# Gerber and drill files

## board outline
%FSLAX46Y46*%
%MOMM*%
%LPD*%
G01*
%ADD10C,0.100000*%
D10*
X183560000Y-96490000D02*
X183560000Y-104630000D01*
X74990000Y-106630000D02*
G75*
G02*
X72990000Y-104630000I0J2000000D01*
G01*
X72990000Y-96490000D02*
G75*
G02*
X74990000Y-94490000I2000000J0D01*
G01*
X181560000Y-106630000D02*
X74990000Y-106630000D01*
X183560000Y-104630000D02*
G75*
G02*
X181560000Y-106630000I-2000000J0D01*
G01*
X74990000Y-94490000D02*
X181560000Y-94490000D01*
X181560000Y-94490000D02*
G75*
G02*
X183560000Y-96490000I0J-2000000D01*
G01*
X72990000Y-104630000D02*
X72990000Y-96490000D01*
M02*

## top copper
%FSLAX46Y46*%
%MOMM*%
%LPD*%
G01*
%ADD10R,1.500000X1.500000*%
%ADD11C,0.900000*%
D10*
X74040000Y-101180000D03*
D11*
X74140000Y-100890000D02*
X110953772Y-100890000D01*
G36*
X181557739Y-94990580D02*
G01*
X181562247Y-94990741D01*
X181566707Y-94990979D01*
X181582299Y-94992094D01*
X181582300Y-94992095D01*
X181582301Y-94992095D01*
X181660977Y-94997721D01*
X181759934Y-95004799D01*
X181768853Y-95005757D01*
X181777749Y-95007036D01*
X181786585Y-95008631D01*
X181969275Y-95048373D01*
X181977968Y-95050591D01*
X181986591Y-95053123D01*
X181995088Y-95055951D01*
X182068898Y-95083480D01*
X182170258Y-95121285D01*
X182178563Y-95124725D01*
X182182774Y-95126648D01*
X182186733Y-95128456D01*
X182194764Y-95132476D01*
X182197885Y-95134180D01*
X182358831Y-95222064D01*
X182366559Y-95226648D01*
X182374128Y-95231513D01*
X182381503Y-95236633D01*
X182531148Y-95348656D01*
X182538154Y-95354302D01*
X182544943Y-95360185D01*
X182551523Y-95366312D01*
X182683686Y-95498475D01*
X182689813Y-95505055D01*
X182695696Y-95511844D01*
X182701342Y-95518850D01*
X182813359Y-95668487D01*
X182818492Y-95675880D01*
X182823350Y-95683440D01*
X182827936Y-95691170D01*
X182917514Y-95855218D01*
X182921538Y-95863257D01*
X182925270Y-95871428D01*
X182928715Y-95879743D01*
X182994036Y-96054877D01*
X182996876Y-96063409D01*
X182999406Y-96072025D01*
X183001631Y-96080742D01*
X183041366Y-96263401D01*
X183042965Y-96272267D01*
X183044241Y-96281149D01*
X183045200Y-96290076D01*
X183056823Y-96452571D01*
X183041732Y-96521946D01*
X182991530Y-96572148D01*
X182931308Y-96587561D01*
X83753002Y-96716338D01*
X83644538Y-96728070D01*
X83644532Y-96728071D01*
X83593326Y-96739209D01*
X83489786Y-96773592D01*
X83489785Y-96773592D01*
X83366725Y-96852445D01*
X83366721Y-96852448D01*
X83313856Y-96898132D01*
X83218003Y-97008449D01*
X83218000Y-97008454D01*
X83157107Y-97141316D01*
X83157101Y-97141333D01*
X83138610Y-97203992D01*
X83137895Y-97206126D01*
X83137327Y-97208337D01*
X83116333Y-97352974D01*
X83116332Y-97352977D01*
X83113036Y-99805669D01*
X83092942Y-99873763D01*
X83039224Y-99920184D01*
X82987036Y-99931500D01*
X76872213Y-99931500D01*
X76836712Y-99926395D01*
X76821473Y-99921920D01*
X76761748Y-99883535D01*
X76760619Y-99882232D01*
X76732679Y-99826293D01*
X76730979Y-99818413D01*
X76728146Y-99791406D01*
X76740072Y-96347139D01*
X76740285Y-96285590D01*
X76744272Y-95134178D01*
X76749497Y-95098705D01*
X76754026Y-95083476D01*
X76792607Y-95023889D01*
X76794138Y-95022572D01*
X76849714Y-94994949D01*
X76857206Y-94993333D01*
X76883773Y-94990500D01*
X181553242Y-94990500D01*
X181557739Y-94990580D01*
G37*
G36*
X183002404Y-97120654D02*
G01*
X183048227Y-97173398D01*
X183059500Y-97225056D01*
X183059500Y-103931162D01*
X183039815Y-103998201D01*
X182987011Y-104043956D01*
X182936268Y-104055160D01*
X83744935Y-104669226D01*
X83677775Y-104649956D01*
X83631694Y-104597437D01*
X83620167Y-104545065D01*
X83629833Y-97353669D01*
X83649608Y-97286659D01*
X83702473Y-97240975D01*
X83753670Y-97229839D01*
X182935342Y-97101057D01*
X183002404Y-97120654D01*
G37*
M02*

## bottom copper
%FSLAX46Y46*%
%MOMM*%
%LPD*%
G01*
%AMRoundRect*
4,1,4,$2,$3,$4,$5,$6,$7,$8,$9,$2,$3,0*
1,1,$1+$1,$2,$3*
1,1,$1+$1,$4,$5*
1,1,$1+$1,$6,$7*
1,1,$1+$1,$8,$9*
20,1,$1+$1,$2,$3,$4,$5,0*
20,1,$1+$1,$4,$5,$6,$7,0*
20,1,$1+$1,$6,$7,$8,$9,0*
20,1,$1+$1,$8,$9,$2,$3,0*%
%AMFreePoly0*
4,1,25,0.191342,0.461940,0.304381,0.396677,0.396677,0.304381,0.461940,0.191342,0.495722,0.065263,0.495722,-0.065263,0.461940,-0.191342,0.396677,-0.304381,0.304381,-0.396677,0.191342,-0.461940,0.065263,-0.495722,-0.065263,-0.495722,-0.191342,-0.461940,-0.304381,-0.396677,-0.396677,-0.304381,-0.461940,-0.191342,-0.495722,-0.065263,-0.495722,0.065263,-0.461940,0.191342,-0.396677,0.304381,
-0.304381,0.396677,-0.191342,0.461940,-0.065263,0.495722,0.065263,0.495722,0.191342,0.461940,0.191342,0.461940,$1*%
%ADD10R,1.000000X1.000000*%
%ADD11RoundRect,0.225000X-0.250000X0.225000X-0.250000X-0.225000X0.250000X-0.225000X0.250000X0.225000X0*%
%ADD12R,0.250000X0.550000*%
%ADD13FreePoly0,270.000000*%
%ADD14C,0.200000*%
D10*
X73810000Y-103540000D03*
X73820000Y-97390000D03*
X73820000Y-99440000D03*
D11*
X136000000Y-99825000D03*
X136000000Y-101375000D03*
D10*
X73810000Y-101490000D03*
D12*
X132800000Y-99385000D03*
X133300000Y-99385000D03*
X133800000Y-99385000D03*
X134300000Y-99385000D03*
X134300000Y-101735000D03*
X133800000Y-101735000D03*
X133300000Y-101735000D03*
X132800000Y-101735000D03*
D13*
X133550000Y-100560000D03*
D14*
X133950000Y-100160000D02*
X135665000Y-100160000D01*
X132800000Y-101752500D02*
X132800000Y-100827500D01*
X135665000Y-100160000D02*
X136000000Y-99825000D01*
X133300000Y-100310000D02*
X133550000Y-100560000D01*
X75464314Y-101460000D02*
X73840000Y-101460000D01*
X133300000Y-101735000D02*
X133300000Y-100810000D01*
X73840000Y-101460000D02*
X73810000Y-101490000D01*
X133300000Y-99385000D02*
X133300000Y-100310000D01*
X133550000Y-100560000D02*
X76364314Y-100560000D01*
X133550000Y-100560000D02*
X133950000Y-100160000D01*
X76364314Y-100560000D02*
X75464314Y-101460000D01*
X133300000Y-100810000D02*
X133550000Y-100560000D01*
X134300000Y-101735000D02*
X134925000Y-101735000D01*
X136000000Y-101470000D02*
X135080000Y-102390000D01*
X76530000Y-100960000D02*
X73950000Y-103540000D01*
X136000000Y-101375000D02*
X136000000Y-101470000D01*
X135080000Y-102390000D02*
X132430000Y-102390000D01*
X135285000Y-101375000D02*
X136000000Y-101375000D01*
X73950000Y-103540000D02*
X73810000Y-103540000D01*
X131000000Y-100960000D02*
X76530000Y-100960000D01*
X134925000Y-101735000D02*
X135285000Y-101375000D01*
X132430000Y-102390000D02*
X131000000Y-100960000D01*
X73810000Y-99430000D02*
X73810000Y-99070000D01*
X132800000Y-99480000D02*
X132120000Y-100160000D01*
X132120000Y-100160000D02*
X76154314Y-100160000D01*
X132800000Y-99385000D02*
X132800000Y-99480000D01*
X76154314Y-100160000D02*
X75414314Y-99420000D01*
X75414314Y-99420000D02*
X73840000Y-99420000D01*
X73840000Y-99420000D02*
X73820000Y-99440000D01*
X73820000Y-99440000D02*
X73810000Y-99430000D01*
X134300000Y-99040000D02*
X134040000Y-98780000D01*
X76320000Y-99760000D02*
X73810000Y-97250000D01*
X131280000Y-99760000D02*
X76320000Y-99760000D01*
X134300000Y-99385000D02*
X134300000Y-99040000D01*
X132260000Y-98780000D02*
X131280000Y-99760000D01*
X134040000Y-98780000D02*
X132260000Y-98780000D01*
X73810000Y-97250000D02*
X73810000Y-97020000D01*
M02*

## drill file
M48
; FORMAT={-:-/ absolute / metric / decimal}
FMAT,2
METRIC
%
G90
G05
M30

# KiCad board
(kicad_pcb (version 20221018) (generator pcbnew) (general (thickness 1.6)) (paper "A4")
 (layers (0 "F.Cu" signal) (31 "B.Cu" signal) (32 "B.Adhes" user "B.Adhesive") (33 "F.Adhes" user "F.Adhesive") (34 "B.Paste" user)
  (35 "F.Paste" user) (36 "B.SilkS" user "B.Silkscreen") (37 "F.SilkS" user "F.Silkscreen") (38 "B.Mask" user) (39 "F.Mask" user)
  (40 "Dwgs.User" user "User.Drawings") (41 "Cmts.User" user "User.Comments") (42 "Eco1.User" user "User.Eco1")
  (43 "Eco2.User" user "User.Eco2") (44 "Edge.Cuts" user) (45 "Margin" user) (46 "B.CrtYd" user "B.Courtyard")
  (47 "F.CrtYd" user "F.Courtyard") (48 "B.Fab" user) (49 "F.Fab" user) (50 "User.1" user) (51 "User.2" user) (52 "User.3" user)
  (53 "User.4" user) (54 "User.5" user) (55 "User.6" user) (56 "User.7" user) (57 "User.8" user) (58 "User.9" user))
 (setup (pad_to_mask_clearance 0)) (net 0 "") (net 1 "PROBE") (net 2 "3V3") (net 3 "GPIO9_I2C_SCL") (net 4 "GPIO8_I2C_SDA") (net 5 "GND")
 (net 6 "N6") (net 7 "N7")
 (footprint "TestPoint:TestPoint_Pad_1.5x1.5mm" (layer "F.Cu") (at 74.04 101.18)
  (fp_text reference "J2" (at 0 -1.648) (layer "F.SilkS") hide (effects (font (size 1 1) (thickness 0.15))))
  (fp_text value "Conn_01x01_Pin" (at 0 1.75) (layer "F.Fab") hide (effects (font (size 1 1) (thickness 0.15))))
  (pad "1" smd rect (at 0 0) (size 1.5 1.5) (layers "F.Cu" "F.Mask") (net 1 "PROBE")))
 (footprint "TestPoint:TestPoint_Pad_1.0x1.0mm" (layer "B.Cu") (at 73.81 103.54 180)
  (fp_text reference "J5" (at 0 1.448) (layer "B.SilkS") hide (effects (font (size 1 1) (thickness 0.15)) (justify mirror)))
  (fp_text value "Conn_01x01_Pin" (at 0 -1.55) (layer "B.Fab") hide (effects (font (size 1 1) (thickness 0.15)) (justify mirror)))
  (pad "1" smd rect (at 0 0 180) (size 1 1) (layers "B.Cu" "B.Mask") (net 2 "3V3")))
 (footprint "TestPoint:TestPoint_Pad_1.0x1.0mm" (layer "B.Cu") (at 73.82 97.39 180)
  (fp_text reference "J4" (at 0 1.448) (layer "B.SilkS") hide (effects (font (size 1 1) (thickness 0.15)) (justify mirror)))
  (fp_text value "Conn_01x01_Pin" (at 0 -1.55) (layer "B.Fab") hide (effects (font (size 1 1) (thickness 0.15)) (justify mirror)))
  (pad "1" smd rect (at 0 0 180) (size 1 1) (layers "B.Cu" "B.Mask") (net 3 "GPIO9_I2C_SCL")))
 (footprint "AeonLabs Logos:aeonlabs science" (layer "B.Cu") (at 174.289702 100.771553)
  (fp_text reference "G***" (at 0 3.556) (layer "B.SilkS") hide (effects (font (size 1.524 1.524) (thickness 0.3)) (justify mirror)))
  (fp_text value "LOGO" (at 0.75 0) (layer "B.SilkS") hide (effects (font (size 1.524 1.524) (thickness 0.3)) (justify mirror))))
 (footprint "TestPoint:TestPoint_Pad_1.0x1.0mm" (layer "B.Cu") (at 73.82 99.44 180)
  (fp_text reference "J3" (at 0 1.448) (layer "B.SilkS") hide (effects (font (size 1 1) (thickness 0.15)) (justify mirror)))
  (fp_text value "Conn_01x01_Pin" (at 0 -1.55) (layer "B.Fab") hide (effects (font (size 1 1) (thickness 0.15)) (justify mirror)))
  (pad "1" smd rect (at 0 0 180) (size 1 1) (layers "B.Cu" "B.Mask") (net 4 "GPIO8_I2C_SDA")))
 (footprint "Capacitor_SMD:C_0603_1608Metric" (layer "B.Cu") (at 136 100.6 -90)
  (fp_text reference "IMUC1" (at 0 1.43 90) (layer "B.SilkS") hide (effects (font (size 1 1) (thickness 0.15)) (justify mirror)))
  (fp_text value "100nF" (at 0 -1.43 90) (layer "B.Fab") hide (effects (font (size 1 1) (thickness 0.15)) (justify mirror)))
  (pad "1" smd roundrect (at -0.775 0 270) (size 0.9 0.95) (layers "B.Cu" "B.Paste" "B.Mask") (roundrect_rratio 0.25) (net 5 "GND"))
  (pad "2" smd roundrect (at 0.775 0 270) (size 0.9 0.95) (layers "B.Cu" "B.Paste" "B.Mask") (roundrect_rratio 0.25) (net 2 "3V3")))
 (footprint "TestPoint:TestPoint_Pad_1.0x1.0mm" (layer "B.Cu") (at 73.81 101.49 180)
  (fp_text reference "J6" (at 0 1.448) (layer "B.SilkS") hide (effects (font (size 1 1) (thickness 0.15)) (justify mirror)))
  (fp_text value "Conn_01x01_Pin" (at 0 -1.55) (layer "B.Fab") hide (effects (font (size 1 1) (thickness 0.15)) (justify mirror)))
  (pad "1" smd rect (at 0 0 180) (size 1 1) (layers "B.Cu" "B.Mask") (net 5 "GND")))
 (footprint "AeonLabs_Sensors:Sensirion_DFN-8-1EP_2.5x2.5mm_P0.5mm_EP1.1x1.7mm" (layer "B.Cu") (at 133.55 100.56 -90)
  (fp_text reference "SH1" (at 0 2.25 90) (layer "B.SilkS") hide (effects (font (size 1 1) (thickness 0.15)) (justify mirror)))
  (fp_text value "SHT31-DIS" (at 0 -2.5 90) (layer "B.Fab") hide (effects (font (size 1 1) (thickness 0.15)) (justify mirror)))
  (pad "" smd custom (at 0 0 270) (size 0.9 0.9) (layers "B.Paste") (zone_connect 0) (thermal_bridge_angle 45)
   (options (clearance outline) (anchor rect)) (primitives))
  (pad "1" smd rect (at -1.175 0.75 270) (size 0.55 0.25) (layers "B.Cu" "B.Paste" "B.Mask") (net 4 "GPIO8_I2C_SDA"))
  (pad "2" smd rect (at -1.175 0.25 270) (size 0.55 0.25) (layers "B.Cu" "B.Paste" "B.Mask") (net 5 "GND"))
  (pad "3" smd rect (at -1.175 -0.25 270) (size 0.55 0.25) (layers "B.Cu" "B.Paste" "B.Mask") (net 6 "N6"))
  (pad "4" smd rect (at -1.175 -0.75 90) (size 0.55 0.25) (layers "B.Cu" "B.Paste" "B.Mask") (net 3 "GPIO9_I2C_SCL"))
  (pad "5" smd rect (at 1.175 -0.75 270) (size 0.55 0.25) (layers "B.Cu" "B.Paste" "B.Mask") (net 2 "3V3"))
  (pad "6" smd rect (at 1.175 -0.25 270) (size 0.55 0.25) (layers "B.Cu" "B.Paste" "B.Mask") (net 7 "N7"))
  (pad "7" smd rect (at 1.175 0.25 270) (size 0.55 0.25) (layers "B.Cu" "B.Paste" "B.Mask") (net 5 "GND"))
  (pad "8" smd rect (at 1.175 0.75 270) (size 0.55 0.25) (layers "B.Cu" "B.Paste" "B.Mask") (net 5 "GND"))
  (pad "9" smd custom (at 0 0 270) (size 1 1) (layers "B.Cu" "B.Mask") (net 5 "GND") (zone_connect 0) (thermal_bridge_angle 45)
   (options (clearance outline) (anchor circle)) (primitives)))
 (gr_line (start 183.56 96.49) (end 183.56 104.63) (stroke (width 0.1) (type default)) (layer "Edge.Cuts"))
 (gr_arc (start 74.99 106.63) (mid 73.575786 106.044214) (end 72.99 104.63) (stroke (width 0.1) (type default)) (layer "Edge.Cuts"))
 (gr_arc (start 72.99 96.49) (mid 73.575786 95.075786) (end 74.99 94.49) (stroke (width 0.1) (type default)) (layer "Edge.Cuts"))
 (gr_line (start 181.56 106.63) (end 74.99 106.63) (stroke (width 0.1) (type default)) (layer "Edge.Cuts"))
 (gr_arc (start 183.56 104.63) (mid 182.974214 106.044214) (end 181.56 106.63) (stroke (width 0.1) (type default)) (layer "Edge.Cuts"))
 (gr_line (start 74.99 94.49) (end 181.56 94.49) (stroke (width 0.1) (type default)) (layer "Edge.Cuts"))
 (gr_arc (start 181.56 94.49) (mid 182.974214 95.075786) (end 183.56 96.49) (stroke (width 0.1) (type default)) (layer "Edge.Cuts"))
 (gr_line (start 72.99 104.63) (end 72.99 96.49) (stroke (width 0.1) (type default)) (layer "Edge.Cuts"))
 (segment (start 74.14 100.89) (end 110.953772 100.89) (width 0.9) (layer "F.Cu") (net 1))
 (segment (start 133.95 100.16) (end 135.665 100.16) (width 0.2) (layer "B.Cu") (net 5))
 (segment (start 132.8 101.7525) (end 132.8 100.8275) (width 0.2) (layer "B.Cu") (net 5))
 (segment (start 135.665 100.16) (end 136 99.825) (width 0.2) (layer "B.Cu") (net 5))
 (segment (start 133.3 100.31) (end 133.55 100.56) (width 0.2) (layer "B.Cu") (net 5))
 (segment (start 75.464314 101.46) (end 73.84 101.46) (width 0.2) (layer "B.Cu") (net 5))
 (segment (start 133.3 101.735) (end 133.3 100.81) (width 0.2) (layer "B.Cu") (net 5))
 (segment (start 73.84 101.46) (end 73.81 101.49) (width 0.2) (layer "B.Cu") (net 5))
 (segment (start 133.3 99.385) (end 133.3 100.31) (width 0.2) (layer "B.Cu") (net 5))
 (segment (start 133.55 100.56) (end 76.364314 100.56) (width 0.2) (layer "B.Cu") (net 5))
 (segment (start 133.55 100.56) (end 133.95 100.16) (width 0.2) (layer "B.Cu") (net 5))
 (segment (start 76.364314 100.56) (end 75.464314 101.46) (width 0.2) (layer "B.Cu") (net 5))
 (segment (start 133.3 100.81) (end 133.55 100.56) (width 0.2) (layer "B.Cu") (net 5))
 (segment (start 134.3 101.735) (end 134.925 101.735) (width 0.2) (layer "B.Cu") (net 2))
 (segment (start 136 101.47) (end 135.08 102.39) (width 0.2) (layer "B.Cu") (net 2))
 (segment (start 76.53 100.96) (end 73.95 103.54) (width 0.2) (layer "B.Cu") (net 2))
 (segment (start 136 101.375) (end 136 101.47) (width 0.2) (layer "B.Cu") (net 2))
 (segment (start 135.08 102.39) (end 132.43 102.39) (width 0.2) (layer "B.Cu") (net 2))
 (segment (start 135.285 101.375) (end 136 101.375) (width 0.2) (layer "B.Cu") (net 2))
 (segment (start 73.95 103.54) (end 73.81 103.54) (width 0.2) (layer "B.Cu") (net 2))
 (segment (start 131 100.96) (end 76.53 100.96) (width 0.2) (layer "B.Cu") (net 2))
 (segment (start 134.925 101.735) (end 135.285 101.375) (width 0.2) (layer "B.Cu") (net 2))
 (segment (start 132.43 102.39) (end 131 100.96) (width 0.2) (layer "B.Cu") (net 2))
 (segment (start 73.81 99.43) (end 73.81 99.07) (width 0.2) (layer "B.Cu") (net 4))
 (segment (start 132.8 99.48) (end 132.12 100.16) (width 0.2) (layer "B.Cu") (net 4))
 (segment (start 132.12 100.16) (end 76.154314 100.16) (width 0.2) (layer "B.Cu") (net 4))
 (segment (start 132.8 99.385) (end 132.8 99.48) (width 0.2) (layer "B.Cu") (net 4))
 (segment (start 76.154314 100.16) (end 75.414314 99.42) (width 0.2) (layer "B.Cu") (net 4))
 (segment (start 75.414314 99.42) (end 73.84 99.42) (width 0.2) (layer "B.Cu") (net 4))
 (segment (start 73.84 99.42) (end 73.82 99.44) (width 0.2) (layer "B.Cu") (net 4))
 (segment (start 73.82 99.44) (end 73.81 99.43) (width 0.2) (layer "B.Cu") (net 4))
 (segment (start 134.3 99.04) (end 134.04 98.78) (width 0.2) (layer "B.Cu") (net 3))
 (segment (start 76.32 99.76) (end 73.81 97.25) (width 0.2) (layer "B.Cu") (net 3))
 (segment (start 131.28 99.76) (end 76.32 99.76) (width 0.2) (layer "B.Cu") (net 3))
 (segment (start 134.3 99.385) (end 134.3 99.04) (width 0.2) (layer "B.Cu") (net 3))
 (segment (start 132.26 98.78) (end 131.28 99.76) (width 0.2) (layer "B.Cu") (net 3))
 (segment (start 134.04 98.78) (end 132.26 98.78) (width 0.2) (layer "B.Cu") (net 3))
 (segment (start 73.81 97.25) (end 73.81 97.02) (width 0.2) (layer "B.Cu") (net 3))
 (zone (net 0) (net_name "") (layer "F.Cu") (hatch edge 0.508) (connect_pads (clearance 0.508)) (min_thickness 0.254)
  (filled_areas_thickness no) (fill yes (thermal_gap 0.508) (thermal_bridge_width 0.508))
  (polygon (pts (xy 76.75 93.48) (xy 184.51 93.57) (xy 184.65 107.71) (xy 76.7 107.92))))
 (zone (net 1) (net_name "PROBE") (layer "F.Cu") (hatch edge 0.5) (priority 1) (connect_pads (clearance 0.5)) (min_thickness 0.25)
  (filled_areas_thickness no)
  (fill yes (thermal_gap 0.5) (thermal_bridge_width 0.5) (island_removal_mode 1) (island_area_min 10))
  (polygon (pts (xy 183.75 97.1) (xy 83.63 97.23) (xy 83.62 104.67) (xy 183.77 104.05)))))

